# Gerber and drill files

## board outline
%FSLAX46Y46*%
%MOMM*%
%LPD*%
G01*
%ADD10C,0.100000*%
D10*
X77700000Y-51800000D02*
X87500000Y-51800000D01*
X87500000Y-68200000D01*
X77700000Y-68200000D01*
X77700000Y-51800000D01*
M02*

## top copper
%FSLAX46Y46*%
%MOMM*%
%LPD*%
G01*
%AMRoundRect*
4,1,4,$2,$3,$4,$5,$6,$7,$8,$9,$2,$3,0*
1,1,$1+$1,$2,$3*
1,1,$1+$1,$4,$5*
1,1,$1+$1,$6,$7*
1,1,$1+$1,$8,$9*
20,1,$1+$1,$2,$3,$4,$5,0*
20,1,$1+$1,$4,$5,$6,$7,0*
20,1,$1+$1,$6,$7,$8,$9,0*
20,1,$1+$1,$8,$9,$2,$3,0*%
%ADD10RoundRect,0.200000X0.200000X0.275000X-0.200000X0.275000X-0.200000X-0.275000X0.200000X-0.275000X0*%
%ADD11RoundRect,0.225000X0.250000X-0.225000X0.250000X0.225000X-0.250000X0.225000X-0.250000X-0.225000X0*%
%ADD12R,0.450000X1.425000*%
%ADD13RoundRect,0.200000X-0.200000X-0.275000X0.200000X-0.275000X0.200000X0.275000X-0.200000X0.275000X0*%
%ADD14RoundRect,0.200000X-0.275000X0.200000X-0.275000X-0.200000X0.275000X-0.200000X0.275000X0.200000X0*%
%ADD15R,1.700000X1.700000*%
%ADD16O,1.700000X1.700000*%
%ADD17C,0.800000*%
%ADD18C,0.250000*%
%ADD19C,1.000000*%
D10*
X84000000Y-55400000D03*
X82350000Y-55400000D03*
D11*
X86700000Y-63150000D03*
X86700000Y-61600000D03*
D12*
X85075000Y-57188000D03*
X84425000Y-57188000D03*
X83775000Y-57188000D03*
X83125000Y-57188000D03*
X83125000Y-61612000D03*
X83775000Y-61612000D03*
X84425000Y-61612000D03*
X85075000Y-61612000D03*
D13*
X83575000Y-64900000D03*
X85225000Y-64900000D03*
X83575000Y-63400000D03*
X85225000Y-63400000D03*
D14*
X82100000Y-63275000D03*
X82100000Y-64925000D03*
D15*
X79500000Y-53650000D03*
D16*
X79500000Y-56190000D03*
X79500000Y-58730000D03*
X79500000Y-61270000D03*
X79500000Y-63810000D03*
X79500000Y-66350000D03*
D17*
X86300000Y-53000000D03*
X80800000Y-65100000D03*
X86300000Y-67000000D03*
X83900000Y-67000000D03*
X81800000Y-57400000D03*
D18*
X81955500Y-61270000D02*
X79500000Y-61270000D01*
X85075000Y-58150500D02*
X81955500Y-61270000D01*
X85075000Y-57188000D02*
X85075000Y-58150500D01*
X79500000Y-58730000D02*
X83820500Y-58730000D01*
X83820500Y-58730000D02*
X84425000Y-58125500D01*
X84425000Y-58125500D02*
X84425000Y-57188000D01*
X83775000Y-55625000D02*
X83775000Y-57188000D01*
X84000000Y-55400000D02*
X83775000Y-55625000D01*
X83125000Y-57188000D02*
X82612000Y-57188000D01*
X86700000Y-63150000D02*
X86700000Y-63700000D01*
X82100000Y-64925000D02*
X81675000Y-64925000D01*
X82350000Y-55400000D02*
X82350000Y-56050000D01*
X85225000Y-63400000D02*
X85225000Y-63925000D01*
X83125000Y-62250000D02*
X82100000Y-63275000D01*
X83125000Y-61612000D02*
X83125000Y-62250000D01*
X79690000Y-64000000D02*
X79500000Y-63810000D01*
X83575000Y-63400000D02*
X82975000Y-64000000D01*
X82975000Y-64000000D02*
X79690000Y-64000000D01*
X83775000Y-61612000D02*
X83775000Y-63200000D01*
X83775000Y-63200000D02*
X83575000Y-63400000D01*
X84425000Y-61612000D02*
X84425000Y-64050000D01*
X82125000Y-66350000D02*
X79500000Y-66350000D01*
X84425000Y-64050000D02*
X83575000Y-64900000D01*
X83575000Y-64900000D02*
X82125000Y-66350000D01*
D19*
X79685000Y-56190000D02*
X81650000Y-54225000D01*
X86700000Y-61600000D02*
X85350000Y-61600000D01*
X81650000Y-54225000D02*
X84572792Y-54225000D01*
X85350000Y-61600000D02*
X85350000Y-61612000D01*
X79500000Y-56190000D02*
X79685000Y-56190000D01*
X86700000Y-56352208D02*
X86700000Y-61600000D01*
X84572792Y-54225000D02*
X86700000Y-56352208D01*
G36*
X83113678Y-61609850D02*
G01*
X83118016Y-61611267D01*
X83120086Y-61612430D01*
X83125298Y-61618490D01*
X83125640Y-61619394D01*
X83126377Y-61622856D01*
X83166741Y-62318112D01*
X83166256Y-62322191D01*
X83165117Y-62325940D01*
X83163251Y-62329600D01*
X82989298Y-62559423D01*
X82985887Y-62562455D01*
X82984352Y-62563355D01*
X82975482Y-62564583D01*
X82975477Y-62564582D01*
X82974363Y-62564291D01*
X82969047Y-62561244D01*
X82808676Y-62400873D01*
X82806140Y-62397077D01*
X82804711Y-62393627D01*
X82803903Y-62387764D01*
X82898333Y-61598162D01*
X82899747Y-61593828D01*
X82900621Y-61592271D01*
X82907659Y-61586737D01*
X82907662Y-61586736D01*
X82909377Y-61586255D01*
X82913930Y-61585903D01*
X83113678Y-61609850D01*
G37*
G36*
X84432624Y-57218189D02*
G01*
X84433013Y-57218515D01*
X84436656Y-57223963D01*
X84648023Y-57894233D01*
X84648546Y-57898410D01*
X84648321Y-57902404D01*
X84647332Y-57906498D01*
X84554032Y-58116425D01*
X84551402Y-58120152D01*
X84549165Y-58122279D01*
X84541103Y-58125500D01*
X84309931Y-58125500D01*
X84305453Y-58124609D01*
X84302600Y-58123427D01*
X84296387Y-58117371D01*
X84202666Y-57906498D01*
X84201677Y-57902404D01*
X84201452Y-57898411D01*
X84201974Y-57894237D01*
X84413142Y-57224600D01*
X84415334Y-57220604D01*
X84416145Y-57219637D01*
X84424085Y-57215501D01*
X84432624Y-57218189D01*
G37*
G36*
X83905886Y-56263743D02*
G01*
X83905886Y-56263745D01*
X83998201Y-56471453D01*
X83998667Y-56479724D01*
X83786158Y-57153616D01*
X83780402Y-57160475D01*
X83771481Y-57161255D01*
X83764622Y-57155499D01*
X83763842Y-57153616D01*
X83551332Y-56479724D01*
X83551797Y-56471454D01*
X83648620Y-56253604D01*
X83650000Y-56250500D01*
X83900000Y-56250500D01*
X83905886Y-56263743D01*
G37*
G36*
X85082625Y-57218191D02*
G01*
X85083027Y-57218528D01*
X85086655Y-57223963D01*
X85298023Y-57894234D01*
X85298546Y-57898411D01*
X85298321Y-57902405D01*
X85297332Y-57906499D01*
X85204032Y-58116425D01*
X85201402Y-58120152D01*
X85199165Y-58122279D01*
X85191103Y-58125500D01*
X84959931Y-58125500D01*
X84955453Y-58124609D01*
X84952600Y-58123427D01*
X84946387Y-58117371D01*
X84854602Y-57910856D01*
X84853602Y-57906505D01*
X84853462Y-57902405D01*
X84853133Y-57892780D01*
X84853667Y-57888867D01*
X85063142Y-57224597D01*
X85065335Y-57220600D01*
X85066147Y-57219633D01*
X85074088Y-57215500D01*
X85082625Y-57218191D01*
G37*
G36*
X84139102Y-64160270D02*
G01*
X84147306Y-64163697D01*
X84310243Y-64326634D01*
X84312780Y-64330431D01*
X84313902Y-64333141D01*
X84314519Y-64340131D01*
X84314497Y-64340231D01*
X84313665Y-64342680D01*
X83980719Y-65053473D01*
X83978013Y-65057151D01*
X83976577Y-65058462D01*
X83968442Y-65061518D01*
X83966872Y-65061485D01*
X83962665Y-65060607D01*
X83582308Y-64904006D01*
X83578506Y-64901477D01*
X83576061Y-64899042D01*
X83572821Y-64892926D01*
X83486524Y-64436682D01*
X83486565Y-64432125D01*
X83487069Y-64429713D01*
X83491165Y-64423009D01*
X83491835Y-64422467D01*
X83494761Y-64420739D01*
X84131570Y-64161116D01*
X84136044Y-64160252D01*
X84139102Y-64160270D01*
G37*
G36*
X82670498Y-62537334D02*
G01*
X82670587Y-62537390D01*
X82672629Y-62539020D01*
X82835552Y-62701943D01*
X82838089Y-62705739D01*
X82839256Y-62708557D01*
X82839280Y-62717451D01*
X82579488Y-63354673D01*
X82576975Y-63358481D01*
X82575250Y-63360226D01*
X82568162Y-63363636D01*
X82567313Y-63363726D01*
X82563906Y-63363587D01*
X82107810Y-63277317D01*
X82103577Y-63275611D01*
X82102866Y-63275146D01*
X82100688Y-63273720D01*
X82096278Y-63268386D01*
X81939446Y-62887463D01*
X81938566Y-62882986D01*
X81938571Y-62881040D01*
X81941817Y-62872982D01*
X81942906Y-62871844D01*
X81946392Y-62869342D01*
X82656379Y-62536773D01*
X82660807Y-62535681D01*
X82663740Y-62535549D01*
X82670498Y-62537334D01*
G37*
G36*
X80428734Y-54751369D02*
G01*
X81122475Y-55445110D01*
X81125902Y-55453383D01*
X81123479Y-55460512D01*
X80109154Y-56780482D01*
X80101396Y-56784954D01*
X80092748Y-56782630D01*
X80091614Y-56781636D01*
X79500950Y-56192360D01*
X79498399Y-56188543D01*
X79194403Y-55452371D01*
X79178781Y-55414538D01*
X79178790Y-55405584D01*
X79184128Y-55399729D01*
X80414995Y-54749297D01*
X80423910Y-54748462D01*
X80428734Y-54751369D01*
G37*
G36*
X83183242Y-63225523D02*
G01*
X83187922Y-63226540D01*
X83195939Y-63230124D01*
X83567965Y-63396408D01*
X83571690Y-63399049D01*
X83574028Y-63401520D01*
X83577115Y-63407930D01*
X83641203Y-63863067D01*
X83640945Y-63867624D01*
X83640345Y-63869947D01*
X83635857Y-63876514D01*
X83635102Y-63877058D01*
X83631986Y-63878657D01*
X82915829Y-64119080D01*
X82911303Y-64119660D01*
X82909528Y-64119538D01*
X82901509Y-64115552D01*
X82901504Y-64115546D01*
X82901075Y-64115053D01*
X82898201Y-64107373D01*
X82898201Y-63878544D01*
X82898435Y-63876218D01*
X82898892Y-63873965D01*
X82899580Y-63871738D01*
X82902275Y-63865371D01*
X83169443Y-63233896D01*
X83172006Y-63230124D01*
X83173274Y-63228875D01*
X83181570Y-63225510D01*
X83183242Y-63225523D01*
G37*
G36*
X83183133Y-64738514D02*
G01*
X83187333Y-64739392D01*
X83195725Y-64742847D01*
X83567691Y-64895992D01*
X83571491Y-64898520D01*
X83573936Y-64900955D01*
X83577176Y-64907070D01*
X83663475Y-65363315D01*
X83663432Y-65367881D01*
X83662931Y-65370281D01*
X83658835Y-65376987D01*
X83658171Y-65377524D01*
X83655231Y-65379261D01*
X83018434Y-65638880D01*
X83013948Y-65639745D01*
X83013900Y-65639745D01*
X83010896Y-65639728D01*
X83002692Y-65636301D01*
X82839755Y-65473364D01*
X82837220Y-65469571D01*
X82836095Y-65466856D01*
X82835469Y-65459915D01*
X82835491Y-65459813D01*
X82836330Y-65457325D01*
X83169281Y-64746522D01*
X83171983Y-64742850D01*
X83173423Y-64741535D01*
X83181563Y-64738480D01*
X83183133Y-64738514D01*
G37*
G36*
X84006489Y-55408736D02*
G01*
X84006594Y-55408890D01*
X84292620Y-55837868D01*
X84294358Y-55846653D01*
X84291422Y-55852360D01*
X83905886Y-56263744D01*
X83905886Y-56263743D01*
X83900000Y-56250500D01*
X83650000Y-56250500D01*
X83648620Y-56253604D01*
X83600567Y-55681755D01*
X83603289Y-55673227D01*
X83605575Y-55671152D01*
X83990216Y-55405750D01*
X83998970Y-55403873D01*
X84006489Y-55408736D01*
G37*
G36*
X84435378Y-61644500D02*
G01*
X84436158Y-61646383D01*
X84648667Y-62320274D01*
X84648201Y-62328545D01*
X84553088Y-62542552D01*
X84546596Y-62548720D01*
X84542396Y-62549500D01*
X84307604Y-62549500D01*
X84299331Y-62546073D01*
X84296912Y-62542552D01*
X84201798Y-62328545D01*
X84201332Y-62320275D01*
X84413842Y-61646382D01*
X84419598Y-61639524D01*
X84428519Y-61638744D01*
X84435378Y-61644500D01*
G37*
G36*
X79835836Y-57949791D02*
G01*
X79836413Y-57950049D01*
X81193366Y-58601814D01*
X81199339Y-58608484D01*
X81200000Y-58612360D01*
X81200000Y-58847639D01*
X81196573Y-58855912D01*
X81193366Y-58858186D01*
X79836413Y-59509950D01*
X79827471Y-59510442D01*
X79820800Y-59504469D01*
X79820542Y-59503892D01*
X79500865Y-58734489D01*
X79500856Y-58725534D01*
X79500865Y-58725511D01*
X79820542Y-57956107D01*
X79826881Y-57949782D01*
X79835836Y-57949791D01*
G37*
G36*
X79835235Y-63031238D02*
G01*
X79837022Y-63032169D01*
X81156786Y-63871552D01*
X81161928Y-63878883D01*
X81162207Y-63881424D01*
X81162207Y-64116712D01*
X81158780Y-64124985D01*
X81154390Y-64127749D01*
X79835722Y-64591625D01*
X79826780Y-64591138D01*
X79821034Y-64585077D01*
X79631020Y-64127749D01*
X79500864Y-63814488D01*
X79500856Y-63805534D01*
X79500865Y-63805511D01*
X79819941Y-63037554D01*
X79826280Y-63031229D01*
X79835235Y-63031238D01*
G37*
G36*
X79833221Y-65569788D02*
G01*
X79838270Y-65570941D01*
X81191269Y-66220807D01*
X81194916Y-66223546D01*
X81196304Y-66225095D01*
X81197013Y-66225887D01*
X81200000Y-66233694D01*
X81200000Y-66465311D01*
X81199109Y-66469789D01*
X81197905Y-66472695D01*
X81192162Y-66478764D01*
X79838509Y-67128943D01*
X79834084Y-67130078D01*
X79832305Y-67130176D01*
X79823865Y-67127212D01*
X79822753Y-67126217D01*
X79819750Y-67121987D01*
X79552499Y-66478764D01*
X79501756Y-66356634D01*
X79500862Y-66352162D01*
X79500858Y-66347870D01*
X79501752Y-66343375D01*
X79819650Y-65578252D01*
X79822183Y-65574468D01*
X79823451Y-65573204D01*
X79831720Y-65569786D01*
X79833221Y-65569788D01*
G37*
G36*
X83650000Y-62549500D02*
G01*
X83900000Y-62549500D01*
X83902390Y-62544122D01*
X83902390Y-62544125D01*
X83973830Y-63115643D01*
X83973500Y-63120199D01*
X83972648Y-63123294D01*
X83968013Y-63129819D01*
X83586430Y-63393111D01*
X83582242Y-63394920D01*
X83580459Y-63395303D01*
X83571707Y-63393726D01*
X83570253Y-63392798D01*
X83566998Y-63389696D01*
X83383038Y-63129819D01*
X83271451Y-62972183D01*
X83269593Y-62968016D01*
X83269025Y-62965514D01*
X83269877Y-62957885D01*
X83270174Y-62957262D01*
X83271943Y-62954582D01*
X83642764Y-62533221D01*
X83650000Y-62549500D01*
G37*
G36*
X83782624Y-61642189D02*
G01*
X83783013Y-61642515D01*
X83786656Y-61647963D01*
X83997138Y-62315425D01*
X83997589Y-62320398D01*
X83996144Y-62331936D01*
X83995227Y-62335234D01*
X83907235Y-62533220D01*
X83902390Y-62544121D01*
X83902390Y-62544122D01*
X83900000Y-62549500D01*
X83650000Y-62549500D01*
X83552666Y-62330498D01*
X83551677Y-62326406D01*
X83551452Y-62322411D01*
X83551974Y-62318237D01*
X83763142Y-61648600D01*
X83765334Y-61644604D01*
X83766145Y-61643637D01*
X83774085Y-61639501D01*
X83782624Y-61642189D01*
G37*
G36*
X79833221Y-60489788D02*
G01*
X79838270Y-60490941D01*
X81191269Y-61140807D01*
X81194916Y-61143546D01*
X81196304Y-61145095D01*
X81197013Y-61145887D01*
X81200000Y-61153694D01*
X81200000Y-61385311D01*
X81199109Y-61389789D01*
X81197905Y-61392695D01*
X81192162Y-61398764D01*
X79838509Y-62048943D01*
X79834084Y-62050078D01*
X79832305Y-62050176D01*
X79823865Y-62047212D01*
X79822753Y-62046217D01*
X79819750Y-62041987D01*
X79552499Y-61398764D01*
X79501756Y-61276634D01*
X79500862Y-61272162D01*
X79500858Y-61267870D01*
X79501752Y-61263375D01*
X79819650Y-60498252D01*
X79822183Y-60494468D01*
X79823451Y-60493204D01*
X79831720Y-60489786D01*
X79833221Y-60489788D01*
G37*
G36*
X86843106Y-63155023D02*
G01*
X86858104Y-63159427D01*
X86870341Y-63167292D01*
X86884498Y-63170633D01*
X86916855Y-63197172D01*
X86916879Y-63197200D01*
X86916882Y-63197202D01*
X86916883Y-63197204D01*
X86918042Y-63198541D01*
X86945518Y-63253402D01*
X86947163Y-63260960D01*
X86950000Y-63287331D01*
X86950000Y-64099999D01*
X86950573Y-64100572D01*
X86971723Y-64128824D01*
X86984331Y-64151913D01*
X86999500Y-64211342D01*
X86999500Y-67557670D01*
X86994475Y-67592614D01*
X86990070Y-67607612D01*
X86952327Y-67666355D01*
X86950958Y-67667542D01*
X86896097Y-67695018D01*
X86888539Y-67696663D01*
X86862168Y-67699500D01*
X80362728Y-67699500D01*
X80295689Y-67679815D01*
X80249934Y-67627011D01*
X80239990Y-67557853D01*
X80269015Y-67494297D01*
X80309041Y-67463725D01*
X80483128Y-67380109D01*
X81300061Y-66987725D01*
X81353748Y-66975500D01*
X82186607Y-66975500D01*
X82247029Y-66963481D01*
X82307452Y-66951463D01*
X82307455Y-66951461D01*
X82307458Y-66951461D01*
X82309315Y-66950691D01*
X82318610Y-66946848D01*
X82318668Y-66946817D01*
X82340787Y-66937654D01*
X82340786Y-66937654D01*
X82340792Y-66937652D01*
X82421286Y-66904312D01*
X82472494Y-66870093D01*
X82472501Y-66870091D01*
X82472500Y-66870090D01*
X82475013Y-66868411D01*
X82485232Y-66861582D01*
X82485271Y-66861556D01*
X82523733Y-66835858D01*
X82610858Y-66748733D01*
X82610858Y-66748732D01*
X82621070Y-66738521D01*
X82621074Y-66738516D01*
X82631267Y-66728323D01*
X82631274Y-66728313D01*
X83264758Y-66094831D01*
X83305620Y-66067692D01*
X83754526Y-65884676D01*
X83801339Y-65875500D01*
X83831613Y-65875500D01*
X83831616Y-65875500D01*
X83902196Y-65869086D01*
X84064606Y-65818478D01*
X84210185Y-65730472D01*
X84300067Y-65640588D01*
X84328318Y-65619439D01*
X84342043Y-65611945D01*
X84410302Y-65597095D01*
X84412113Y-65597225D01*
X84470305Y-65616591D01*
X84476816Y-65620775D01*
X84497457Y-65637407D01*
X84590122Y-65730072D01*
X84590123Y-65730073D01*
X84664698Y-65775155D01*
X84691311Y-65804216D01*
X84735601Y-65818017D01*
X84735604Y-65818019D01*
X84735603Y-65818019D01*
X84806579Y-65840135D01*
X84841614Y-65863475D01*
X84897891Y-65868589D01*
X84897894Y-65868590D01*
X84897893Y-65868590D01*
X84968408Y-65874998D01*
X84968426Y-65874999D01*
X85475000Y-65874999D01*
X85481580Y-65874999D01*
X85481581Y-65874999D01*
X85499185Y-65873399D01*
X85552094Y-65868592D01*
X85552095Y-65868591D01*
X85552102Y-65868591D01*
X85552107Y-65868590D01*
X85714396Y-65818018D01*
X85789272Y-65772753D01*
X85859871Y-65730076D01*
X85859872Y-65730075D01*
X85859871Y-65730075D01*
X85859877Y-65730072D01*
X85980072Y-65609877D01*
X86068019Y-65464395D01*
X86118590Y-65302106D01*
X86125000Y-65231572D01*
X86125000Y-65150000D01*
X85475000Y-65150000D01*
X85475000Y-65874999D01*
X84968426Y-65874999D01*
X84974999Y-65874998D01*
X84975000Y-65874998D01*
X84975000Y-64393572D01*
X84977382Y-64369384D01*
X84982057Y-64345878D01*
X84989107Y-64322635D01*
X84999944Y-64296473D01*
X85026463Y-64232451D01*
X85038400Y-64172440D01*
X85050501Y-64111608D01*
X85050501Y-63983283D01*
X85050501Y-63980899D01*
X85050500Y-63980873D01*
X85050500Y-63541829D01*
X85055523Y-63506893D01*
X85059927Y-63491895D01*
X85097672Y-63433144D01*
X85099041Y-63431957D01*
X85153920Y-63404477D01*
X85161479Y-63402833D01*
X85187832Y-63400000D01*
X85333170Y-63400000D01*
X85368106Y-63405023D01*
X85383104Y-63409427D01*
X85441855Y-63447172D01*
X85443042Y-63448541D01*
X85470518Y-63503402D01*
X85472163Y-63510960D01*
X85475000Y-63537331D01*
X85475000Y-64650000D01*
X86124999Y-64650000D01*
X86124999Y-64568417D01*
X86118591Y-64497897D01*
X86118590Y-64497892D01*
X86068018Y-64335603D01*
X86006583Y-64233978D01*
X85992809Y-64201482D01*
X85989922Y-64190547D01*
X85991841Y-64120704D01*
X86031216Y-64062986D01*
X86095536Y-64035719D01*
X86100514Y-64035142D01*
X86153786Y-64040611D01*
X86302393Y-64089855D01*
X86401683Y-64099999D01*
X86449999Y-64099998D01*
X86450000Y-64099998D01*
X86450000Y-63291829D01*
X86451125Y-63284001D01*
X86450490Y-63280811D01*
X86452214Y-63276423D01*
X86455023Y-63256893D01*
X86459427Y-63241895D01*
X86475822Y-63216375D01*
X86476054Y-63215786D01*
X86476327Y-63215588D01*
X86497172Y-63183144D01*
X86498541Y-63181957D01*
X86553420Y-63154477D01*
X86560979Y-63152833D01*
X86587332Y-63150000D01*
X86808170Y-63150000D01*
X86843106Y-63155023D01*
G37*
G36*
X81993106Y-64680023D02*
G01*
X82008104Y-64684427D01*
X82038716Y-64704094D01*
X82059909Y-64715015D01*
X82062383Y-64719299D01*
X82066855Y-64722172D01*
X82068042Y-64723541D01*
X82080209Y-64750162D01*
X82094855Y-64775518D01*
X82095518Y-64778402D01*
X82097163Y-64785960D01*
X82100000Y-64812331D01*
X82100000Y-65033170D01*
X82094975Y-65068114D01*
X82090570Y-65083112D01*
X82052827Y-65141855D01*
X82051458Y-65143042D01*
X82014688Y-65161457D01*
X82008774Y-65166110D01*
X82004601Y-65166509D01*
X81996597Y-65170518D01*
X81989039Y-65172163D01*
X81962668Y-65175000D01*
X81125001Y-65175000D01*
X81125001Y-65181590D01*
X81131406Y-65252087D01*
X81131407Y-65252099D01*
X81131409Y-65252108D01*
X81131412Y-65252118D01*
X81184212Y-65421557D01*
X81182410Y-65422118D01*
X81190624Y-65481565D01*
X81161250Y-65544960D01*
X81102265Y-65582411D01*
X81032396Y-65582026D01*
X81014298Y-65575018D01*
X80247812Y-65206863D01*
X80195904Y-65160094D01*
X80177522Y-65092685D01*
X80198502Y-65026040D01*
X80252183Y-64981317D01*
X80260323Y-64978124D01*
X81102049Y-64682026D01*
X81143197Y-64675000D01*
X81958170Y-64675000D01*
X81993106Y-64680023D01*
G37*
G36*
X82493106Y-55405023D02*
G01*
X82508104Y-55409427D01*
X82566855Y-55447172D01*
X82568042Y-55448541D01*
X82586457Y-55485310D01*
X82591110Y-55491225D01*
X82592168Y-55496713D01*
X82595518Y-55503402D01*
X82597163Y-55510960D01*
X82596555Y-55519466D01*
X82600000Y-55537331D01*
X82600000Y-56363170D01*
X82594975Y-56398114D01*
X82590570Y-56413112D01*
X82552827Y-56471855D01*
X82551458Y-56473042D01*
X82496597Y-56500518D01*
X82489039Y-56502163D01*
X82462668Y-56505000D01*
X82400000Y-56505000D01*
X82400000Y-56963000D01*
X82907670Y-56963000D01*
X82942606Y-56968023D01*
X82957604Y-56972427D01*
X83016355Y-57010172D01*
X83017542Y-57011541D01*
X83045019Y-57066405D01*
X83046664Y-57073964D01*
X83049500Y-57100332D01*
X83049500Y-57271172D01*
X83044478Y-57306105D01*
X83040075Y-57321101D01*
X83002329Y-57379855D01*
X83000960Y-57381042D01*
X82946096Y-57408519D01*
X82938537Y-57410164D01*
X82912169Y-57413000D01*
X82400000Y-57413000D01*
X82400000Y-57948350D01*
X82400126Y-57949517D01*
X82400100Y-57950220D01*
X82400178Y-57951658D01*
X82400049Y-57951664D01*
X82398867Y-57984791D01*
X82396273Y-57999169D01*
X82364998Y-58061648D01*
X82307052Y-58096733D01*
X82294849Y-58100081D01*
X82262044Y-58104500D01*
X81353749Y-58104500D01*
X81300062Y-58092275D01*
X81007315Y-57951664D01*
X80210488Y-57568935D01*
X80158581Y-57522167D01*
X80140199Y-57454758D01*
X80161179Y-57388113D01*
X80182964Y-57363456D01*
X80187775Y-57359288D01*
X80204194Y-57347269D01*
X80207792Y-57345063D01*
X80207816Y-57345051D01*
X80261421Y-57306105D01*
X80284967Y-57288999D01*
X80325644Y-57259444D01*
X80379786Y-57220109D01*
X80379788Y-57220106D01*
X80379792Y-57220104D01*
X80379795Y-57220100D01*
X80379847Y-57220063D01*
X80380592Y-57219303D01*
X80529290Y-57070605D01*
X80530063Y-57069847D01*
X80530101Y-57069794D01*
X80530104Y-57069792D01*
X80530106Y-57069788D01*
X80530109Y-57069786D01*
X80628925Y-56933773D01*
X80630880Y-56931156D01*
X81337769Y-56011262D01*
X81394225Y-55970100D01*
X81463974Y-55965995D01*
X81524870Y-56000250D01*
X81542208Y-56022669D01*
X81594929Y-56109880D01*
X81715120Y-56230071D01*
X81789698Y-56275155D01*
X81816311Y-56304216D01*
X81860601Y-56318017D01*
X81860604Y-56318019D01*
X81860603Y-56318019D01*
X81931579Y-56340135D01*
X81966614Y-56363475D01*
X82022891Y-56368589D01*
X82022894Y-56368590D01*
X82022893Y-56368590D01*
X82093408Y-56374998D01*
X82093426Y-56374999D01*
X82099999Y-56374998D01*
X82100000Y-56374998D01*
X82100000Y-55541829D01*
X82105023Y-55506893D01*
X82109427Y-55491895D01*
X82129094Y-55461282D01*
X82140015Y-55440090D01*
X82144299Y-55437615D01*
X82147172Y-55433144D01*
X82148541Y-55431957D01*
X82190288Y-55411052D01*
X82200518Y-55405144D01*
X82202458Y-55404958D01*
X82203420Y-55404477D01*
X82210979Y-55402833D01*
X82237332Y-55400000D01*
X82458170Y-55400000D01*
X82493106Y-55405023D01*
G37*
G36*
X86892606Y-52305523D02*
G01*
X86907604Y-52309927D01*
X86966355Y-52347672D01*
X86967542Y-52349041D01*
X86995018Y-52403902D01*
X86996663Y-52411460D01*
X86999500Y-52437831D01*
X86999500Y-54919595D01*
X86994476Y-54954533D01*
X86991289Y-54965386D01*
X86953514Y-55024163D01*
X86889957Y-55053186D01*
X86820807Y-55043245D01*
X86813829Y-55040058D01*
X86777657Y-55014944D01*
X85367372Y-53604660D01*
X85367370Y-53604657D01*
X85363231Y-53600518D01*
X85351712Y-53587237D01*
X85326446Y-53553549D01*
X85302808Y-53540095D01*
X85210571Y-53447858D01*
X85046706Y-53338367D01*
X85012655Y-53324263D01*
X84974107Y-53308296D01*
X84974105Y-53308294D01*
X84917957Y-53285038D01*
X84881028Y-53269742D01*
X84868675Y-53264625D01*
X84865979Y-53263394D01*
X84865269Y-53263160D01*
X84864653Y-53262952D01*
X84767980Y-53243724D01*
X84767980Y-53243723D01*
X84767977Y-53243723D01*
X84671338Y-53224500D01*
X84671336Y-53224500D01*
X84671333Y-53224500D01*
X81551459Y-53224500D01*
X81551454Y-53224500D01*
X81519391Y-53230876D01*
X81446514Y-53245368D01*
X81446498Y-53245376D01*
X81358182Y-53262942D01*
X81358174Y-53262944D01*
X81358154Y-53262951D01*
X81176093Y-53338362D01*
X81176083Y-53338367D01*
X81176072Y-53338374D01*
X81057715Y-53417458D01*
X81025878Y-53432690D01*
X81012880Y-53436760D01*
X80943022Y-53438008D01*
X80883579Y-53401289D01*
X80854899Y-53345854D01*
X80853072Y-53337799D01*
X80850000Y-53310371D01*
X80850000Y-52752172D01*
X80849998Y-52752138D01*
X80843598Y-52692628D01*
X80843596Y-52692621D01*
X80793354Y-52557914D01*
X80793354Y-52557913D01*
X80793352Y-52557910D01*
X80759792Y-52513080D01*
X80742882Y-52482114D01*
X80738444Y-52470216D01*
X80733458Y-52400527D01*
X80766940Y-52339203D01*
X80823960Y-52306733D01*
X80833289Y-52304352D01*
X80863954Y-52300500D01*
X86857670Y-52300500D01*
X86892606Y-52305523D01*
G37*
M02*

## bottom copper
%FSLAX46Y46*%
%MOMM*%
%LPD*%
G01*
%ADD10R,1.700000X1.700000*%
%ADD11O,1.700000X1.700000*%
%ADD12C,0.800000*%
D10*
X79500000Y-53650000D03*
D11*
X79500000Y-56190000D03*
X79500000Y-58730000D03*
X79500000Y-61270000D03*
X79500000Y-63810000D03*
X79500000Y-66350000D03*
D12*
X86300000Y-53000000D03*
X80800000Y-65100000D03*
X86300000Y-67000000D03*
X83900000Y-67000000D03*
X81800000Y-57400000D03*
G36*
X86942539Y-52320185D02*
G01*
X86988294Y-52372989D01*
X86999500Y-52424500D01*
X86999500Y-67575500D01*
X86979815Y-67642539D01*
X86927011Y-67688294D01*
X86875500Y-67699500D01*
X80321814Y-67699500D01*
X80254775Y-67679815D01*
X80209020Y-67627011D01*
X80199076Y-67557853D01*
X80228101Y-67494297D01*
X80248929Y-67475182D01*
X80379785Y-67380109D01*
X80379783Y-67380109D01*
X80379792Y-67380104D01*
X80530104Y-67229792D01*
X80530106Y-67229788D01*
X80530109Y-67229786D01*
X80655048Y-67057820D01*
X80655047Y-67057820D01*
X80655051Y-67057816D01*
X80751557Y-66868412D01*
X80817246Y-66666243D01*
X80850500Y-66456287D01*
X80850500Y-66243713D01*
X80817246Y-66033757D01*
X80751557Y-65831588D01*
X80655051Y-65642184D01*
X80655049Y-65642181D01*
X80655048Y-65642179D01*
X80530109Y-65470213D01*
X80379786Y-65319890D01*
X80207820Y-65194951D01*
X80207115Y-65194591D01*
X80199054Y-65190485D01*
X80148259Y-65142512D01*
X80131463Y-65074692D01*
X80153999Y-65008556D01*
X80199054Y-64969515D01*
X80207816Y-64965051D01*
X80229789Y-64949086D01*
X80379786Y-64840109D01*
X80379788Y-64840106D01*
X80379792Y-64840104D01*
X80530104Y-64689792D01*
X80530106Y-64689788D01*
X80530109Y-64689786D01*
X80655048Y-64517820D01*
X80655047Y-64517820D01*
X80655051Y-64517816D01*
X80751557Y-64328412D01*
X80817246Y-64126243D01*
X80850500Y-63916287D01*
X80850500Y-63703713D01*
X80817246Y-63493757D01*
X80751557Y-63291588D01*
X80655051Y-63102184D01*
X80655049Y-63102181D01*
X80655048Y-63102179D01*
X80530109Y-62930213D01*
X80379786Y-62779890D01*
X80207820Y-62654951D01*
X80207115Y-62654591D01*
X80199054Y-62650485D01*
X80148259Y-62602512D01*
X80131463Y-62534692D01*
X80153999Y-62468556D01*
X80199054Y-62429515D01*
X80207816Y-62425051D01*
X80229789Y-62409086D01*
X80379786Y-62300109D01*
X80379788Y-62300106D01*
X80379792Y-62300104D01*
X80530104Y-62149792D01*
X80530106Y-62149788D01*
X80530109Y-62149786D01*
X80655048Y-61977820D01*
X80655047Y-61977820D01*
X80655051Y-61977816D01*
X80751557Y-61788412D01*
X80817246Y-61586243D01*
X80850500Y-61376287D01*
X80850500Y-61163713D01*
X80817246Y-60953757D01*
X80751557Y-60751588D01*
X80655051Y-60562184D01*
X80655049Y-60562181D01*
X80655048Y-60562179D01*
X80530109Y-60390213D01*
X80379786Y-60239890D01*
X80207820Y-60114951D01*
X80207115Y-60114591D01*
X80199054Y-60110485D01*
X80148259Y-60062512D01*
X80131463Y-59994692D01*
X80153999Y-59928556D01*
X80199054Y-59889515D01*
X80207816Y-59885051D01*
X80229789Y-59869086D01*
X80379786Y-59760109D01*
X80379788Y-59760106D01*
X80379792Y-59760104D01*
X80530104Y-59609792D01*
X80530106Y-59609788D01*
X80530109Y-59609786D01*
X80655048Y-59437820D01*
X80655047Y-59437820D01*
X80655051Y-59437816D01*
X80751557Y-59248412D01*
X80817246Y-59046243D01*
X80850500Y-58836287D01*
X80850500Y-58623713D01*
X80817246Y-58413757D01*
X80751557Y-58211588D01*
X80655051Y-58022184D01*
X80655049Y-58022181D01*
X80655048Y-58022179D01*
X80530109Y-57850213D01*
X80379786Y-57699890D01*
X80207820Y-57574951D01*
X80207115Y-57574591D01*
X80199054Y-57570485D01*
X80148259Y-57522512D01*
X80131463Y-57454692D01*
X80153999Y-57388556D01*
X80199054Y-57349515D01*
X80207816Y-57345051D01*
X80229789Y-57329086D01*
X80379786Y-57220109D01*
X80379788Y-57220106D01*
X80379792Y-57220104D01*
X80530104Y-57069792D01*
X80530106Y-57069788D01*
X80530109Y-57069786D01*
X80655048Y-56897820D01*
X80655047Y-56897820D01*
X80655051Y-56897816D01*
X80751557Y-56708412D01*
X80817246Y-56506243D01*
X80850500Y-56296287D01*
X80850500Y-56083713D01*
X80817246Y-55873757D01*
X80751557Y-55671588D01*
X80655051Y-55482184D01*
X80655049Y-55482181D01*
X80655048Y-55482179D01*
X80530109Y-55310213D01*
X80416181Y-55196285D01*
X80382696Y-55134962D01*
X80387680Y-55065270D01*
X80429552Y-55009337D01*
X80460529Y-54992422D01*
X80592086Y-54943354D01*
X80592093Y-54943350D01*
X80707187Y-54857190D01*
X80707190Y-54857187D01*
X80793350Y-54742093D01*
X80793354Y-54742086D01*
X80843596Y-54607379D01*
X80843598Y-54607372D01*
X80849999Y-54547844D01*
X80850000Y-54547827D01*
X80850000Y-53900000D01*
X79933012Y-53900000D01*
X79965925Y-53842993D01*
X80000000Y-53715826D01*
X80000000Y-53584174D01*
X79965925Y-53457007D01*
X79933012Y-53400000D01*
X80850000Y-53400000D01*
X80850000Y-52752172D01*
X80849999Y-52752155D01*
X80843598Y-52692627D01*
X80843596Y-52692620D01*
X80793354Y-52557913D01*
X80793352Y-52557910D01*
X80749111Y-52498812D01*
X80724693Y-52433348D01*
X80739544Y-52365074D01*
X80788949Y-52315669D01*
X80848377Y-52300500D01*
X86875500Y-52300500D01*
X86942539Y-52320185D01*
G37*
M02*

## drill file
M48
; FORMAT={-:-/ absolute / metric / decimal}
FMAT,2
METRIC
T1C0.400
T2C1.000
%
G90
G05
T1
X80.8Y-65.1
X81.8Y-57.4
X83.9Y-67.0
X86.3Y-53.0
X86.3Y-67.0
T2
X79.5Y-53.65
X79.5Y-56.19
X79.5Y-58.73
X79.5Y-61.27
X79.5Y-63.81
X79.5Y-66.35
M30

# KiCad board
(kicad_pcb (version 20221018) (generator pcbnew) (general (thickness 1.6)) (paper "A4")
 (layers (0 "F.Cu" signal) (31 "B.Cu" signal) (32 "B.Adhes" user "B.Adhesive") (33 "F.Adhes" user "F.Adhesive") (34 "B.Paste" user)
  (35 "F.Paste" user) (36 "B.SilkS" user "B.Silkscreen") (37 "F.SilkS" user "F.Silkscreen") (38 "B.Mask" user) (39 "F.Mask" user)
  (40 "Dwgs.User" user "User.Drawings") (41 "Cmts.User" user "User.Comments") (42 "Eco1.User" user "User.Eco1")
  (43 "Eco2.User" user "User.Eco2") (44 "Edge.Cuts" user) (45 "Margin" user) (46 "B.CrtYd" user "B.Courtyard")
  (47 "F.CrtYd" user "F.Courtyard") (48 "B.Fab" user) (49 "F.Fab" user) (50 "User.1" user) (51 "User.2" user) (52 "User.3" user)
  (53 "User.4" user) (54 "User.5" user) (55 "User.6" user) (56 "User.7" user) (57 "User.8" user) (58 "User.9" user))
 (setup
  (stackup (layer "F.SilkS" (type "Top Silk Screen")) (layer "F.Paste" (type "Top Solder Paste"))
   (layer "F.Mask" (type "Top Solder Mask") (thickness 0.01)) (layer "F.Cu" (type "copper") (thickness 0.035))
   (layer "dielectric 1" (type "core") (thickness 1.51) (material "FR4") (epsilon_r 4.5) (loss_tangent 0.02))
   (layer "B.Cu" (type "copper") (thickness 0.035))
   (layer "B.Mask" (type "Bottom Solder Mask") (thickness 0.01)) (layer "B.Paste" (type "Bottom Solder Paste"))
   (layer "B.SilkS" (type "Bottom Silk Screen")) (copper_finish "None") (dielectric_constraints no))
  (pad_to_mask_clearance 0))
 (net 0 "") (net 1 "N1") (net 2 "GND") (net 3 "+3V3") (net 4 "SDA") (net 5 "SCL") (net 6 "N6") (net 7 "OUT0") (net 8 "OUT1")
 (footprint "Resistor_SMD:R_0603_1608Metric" (layer "F.Cu") (at 83.175 55.4 180)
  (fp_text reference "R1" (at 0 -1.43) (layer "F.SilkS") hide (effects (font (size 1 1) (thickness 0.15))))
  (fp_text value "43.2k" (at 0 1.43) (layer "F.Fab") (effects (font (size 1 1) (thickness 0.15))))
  (pad "1" smd roundrect (at -0.825 0 180) (size 0.8 0.95) (layers "F.Cu" "F.Paste" "F.Mask") (roundrect_rratio 0.25) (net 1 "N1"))
  (pad "2" smd roundrect (at 0.825 0 180) (size 0.8 0.95) (layers "F.Cu" "F.Paste" "F.Mask") (roundrect_rratio 0.25) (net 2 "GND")))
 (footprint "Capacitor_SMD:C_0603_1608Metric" (layer "F.Cu") (at 86.7 62.375 90)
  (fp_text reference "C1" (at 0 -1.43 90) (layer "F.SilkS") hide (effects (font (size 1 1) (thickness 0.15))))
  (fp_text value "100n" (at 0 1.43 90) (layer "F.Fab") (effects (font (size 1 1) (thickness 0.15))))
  (pad "1" smd roundrect (at -0.775 0 90) (size 0.9 0.95) (layers "F.Cu" "F.Paste" "F.Mask") (roundrect_rratio 0.25) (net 2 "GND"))
  (pad "2" smd roundrect (at 0.775 0 90) (size 0.9 0.95) (layers "F.Cu" "F.Paste" "F.Mask") (roundrect_rratio 0.25) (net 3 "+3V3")))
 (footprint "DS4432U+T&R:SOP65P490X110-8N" (layer "F.Cu") (at 84.1 59.4 -90)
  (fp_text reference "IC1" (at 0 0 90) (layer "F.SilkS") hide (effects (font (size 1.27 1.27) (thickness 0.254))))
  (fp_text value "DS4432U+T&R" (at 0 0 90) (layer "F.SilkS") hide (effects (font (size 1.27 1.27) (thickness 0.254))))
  (pad "1" smd rect (at -2.212 -0.975) (size 0.45 1.425) (layers "F.Cu" "F.Paste" "F.Mask") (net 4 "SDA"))
  (pad "2" smd rect (at -2.212 -0.325) (size 0.45 1.425) (layers "F.Cu" "F.Paste" "F.Mask") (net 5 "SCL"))
  (pad "3" smd rect (at -2.212 0.325) (size 0.45 1.425) (layers "F.Cu" "F.Paste" "F.Mask") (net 1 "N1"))
  (pad "4" smd rect (at -2.212 0.975) (size 0.45 1.425) (layers "F.Cu" "F.Paste" "F.Mask") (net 2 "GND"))
  (pad "5" smd rect (at 2.212 0.975) (size 0.45 1.425) (layers "F.Cu" "F.Paste" "F.Mask") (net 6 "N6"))
  (pad "6" smd rect (at 2.212 0.325) (size 0.45 1.425) (layers "F.Cu" "F.Paste" "F.Mask") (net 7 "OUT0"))
  (pad "7" smd rect (at 2.212 -0.325) (size 0.45 1.425) (layers "F.Cu" "F.Paste" "F.Mask") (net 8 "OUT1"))
  (pad "8" smd rect (at 2.212 -0.975) (size 0.45 1.425) (layers "F.Cu" "F.Paste" "F.Mask") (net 3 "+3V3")))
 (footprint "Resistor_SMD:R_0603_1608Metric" (layer "F.Cu") (at 84.4 64.9)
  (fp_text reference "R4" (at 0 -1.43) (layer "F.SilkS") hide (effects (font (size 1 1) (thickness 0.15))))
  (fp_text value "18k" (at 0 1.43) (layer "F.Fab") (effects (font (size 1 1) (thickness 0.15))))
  (pad "1" smd roundrect (at -0.825 0) (size 0.8 0.95) (layers "F.Cu" "F.Paste" "F.Mask") (roundrect_rratio 0.25) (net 8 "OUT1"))
  (pad "2" smd roundrect (at 0.825 0) (size 0.8 0.95) (layers "F.Cu" "F.Paste" "F.Mask") (roundrect_rratio 0.25) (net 2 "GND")))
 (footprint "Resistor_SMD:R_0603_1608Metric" (layer "F.Cu") (at 84.4 63.4)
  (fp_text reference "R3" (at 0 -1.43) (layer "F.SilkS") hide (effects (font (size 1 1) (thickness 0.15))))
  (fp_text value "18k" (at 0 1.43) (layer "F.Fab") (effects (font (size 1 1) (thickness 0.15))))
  (pad "1" smd roundrect (at -0.825 0) (size 0.8 0.95) (layers "F.Cu" "F.Paste" "F.Mask") (roundrect_rratio 0.25) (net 7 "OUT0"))
  (pad "2" smd roundrect (at 0.825 0) (size 0.8 0.95) (layers "F.Cu" "F.Paste" "F.Mask") (roundrect_rratio 0.25) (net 2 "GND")))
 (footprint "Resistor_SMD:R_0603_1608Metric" (layer "F.Cu") (at 82.1 64.1 -90)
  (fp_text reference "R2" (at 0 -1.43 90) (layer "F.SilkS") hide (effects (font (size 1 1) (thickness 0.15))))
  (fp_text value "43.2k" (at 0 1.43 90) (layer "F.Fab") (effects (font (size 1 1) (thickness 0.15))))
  (pad "1" smd roundrect (at -0.825 0 270) (size 0.8 0.95) (layers "F.Cu" "F.Paste" "F.Mask") (roundrect_rratio 0.25) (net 6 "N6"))
  (pad "2" smd roundrect (at 0.825 0 270) (size 0.8 0.95) (layers "F.Cu" "F.Paste" "F.Mask") (roundrect_rratio 0.25) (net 2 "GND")))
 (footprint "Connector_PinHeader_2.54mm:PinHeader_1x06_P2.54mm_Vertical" (layer "B.Cu") (at 79.5 53.65 180)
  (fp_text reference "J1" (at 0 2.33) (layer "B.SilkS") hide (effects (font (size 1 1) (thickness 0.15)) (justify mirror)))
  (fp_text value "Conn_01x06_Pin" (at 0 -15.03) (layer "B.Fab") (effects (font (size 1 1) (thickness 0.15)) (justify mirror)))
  (pad "1" thru_hole rect (at 0 0 180) (size 1.7 1.7) (drill 1) (layers "*.Cu" "*.Mask") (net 2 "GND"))
  (pad "2" thru_hole oval (at 0 -2.54 180) (size 1.7 1.7) (drill 1) (layers "*.Cu" "*.Mask") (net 3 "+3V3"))
  (pad "3" thru_hole oval (at 0 -5.08 180) (size 1.7 1.7) (drill 1) (layers "*.Cu" "*.Mask") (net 5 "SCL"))
  (pad "4" thru_hole oval (at 0 -7.62 180) (size 1.7 1.7) (drill 1) (layers "*.Cu" "*.Mask") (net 4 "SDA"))
  (pad "5" thru_hole oval (at 0 -10.16 180) (size 1.7 1.7) (drill 1) (layers "*.Cu" "*.Mask") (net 7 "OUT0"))
  (pad "6" thru_hole oval (at 0 -12.7 180) (size 1.7 1.7) (drill 1) (layers "*.Cu" "*.Mask") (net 8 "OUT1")))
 (gr_rect (start 77.7 51.8) (end 87.5 68.2) (stroke (width 0.1) (type default)) (fill none) (layer "Edge.Cuts"))
 (segment (start 81.9555 61.27) (end 79.5 61.27) (width 0.25) (layer "F.Cu") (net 4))
 (segment (start 85.075 58.1505) (end 81.9555 61.27) (width 0.25) (layer "F.Cu") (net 4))
 (segment (start 85.075 57.188) (end 85.075 58.1505) (width 0.25) (layer "F.Cu") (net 4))
 (segment (start 79.5 58.73) (end 83.8205 58.73) (width 0.25) (layer "F.Cu") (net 5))
 (segment (start 83.8205 58.73) (end 84.425 58.1255) (width 0.25) (layer "F.Cu") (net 5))
 (segment (start 84.425 58.1255) (end 84.425 57.188) (width 0.25) (layer "F.Cu") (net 5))
 (segment (start 83.775 55.625) (end 83.775 57.188) (width 0.25) (layer "F.Cu") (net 1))
 (segment (start 84 55.4) (end 83.775 55.625) (width 0.25) (layer "F.Cu") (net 1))
 (segment (start 83.125 57.188) (end 82.612 57.188) (width 0.25) (layer "F.Cu") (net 2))
 (segment (start 86.7 63.15) (end 86.7 63.7) (width 0.25) (layer "F.Cu") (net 2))
 (segment (start 82.1 64.925) (end 81.675 64.925) (width 0.25) (layer "F.Cu") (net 2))
 (segment (start 82.35 55.4) (end 82.35 56.05) (width 0.25) (layer "F.Cu") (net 2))
 (segment (start 85.225 63.4) (end 85.225 63.925) (width 0.25) (layer "F.Cu") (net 2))
 (via (at 86.3 53) (size 0.8) (drill 0.4) (layers "F.Cu" "B.Cu") (free) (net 2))
 (via (at 80.8 65.1) (size 0.8) (drill 0.4) (layers "F.Cu" "B.Cu") (free) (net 2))
 (via (at 86.3 67) (size 0.8) (drill 0.4) (layers "F.Cu" "B.Cu") (free) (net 2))
 (via (at 83.9 67) (size 0.8) (drill 0.4) (layers "F.Cu" "B.Cu") (free) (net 2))
 (via (at 81.8 57.4) (size 0.8) (drill 0.4) (layers "F.Cu" "B.Cu") (free) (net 2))
 (segment (start 83.125 62.25) (end 82.1 63.275) (width 0.25) (layer "F.Cu") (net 6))
 (segment (start 83.125 61.612) (end 83.125 62.25) (width 0.25) (layer "F.Cu") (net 6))
 (segment (start 79.69 64) (end 79.5 63.81) (width 0.25) (layer "F.Cu") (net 7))
 (segment (start 83.575 63.4) (end 82.975 64) (width 0.25) (layer "F.Cu") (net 7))
 (segment (start 82.975 64) (end 79.69 64) (width 0.25) (layer "F.Cu") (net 7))
 (segment (start 83.775 61.612) (end 83.775 63.2) (width 0.25) (layer "F.Cu") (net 7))
 (segment (start 83.775 63.2) (end 83.575 63.4) (width 0.25) (layer "F.Cu") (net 7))
 (segment (start 84.425 61.612) (end 84.425 64.05) (width 0.25) (layer "F.Cu") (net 8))
 (segment (start 82.125 66.35) (end 79.5 66.35) (width 0.25) (layer "F.Cu") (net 8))
 (segment (start 84.425 64.05) (end 83.575 64.9) (width 0.25) (layer "F.Cu") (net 8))
 (segment (start 83.575 64.9) (end 82.125 66.35) (width 0.25) (layer "F.Cu") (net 8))
 (segment (start 79.685 56.19) (end 81.65 54.225) (width 1) (layer "F.Cu") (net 3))
 (segment (start 86.7 61.6) (end 85.35 61.6) (width 1) (layer "F.Cu") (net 3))
 (segment (start 81.65 54.225) (end 84.572792 54.225) (width 1) (layer "F.Cu") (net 3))
 (segment (start 85.35 61.6) (end 85.35 61.612) (width 1) (layer "F.Cu") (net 3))
 (segment (start 79.5 56.19) (end 79.685 56.19) (width 1) (layer "F.Cu") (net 3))
 (segment (start 86.7 56.352208) (end 86.7 61.6) (width 1) (layer "F.Cu") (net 3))
 (segment (start 84.572792 54.225) (end 86.7 56.352208) (width 1) (layer "F.Cu") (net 3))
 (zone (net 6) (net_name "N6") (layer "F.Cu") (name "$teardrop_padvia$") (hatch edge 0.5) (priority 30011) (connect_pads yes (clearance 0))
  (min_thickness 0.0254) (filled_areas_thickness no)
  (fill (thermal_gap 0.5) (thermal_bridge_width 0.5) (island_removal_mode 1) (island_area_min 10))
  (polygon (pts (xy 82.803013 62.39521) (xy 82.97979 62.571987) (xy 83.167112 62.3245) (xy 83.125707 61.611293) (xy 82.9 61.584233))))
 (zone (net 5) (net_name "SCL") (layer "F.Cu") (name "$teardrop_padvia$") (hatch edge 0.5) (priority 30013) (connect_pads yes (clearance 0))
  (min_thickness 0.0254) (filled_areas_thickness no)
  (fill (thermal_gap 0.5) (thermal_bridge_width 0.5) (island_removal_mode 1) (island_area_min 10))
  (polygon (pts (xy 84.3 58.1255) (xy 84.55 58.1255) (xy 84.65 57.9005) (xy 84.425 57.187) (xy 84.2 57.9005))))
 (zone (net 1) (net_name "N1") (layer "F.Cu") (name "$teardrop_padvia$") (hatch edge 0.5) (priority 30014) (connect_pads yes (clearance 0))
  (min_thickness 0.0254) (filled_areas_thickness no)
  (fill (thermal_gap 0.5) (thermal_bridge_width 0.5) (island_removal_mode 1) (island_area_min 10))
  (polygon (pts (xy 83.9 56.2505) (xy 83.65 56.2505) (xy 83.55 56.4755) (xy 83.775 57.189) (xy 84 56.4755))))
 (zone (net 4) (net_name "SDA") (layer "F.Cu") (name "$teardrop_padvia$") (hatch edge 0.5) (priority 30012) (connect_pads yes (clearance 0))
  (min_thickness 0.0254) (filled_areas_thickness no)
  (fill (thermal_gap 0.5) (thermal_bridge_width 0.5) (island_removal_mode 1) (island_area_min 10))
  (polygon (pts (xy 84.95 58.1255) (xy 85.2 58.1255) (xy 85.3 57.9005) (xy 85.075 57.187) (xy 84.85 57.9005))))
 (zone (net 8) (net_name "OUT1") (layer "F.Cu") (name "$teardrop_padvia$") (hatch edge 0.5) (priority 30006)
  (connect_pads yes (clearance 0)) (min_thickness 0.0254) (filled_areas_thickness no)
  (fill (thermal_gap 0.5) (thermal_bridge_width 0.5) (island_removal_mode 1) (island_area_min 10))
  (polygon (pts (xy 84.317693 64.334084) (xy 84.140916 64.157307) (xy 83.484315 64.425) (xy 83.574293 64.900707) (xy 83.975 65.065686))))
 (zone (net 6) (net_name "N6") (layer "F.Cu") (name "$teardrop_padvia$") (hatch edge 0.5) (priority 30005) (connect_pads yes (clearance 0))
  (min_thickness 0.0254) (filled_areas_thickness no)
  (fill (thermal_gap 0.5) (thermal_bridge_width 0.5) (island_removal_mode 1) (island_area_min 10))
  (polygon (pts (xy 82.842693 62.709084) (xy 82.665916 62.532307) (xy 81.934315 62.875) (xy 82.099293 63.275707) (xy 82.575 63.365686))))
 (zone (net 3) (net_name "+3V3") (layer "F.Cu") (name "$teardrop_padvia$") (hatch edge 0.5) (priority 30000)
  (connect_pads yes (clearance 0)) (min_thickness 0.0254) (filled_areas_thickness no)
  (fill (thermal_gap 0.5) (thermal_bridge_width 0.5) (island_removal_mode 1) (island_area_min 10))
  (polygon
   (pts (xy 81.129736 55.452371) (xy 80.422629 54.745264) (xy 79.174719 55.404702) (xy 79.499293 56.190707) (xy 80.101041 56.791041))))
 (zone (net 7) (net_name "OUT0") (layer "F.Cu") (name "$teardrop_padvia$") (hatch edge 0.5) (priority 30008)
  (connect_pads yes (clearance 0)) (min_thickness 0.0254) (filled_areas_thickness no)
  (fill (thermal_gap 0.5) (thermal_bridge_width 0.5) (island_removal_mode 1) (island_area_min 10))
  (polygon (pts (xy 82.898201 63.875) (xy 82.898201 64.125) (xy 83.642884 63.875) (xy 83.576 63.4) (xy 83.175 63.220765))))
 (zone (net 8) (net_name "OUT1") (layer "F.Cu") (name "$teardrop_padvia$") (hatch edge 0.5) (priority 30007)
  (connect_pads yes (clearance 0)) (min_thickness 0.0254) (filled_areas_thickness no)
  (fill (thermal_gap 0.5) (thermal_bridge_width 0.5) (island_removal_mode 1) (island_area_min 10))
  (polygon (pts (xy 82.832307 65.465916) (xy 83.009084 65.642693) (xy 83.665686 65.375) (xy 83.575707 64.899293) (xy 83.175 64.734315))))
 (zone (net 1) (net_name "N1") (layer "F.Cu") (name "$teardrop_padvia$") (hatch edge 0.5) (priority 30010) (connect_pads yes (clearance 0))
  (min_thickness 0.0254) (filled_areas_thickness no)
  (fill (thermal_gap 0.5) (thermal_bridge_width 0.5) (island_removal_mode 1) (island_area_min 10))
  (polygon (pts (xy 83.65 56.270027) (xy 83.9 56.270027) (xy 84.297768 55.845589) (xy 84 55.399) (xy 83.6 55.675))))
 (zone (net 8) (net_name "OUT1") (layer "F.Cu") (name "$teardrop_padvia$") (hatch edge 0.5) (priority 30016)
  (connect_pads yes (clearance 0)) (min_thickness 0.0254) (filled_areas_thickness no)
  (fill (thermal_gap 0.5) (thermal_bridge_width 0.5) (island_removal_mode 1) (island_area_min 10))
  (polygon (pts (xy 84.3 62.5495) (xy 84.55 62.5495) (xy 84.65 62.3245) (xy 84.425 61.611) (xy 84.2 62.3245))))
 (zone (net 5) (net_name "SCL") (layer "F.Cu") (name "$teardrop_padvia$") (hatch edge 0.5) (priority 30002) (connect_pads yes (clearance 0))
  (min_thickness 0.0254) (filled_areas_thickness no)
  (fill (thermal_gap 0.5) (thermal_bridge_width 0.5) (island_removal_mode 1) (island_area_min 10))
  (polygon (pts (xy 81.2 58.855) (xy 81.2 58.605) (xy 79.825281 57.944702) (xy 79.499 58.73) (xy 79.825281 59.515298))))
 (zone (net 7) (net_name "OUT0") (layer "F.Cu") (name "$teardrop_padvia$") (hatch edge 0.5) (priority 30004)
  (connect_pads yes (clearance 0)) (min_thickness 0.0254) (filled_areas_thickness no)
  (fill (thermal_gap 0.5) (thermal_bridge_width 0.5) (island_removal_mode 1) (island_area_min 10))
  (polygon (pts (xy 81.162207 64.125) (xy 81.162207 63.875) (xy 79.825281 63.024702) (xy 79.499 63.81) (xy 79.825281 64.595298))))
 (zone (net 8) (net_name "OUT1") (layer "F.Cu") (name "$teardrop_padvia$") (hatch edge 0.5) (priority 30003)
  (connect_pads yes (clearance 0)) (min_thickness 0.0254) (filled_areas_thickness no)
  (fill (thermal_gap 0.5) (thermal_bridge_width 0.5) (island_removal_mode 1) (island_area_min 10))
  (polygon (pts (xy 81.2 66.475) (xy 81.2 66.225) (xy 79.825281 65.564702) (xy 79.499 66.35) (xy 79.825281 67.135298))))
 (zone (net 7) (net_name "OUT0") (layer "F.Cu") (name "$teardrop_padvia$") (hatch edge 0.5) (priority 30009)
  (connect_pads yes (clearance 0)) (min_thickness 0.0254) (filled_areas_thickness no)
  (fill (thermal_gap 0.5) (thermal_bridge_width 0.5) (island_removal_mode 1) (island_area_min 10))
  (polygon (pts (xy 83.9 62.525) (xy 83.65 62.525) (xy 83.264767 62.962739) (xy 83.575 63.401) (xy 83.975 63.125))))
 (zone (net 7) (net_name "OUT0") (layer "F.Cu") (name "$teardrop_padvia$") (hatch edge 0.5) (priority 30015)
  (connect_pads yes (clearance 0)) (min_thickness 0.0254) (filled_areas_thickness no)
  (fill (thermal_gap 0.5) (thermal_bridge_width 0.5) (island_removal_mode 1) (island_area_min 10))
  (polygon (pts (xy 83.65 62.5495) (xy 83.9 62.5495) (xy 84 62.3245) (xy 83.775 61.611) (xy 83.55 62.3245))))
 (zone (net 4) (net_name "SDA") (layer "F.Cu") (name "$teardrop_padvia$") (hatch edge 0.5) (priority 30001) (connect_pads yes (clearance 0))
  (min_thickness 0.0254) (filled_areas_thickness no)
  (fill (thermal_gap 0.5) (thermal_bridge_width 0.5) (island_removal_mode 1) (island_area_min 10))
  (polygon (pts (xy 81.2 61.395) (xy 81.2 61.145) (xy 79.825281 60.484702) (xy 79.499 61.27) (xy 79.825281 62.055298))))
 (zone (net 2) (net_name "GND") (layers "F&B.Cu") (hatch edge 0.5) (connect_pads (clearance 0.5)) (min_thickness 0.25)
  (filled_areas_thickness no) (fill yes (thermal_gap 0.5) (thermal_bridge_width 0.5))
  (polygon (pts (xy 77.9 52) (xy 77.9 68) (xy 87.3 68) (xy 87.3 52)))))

